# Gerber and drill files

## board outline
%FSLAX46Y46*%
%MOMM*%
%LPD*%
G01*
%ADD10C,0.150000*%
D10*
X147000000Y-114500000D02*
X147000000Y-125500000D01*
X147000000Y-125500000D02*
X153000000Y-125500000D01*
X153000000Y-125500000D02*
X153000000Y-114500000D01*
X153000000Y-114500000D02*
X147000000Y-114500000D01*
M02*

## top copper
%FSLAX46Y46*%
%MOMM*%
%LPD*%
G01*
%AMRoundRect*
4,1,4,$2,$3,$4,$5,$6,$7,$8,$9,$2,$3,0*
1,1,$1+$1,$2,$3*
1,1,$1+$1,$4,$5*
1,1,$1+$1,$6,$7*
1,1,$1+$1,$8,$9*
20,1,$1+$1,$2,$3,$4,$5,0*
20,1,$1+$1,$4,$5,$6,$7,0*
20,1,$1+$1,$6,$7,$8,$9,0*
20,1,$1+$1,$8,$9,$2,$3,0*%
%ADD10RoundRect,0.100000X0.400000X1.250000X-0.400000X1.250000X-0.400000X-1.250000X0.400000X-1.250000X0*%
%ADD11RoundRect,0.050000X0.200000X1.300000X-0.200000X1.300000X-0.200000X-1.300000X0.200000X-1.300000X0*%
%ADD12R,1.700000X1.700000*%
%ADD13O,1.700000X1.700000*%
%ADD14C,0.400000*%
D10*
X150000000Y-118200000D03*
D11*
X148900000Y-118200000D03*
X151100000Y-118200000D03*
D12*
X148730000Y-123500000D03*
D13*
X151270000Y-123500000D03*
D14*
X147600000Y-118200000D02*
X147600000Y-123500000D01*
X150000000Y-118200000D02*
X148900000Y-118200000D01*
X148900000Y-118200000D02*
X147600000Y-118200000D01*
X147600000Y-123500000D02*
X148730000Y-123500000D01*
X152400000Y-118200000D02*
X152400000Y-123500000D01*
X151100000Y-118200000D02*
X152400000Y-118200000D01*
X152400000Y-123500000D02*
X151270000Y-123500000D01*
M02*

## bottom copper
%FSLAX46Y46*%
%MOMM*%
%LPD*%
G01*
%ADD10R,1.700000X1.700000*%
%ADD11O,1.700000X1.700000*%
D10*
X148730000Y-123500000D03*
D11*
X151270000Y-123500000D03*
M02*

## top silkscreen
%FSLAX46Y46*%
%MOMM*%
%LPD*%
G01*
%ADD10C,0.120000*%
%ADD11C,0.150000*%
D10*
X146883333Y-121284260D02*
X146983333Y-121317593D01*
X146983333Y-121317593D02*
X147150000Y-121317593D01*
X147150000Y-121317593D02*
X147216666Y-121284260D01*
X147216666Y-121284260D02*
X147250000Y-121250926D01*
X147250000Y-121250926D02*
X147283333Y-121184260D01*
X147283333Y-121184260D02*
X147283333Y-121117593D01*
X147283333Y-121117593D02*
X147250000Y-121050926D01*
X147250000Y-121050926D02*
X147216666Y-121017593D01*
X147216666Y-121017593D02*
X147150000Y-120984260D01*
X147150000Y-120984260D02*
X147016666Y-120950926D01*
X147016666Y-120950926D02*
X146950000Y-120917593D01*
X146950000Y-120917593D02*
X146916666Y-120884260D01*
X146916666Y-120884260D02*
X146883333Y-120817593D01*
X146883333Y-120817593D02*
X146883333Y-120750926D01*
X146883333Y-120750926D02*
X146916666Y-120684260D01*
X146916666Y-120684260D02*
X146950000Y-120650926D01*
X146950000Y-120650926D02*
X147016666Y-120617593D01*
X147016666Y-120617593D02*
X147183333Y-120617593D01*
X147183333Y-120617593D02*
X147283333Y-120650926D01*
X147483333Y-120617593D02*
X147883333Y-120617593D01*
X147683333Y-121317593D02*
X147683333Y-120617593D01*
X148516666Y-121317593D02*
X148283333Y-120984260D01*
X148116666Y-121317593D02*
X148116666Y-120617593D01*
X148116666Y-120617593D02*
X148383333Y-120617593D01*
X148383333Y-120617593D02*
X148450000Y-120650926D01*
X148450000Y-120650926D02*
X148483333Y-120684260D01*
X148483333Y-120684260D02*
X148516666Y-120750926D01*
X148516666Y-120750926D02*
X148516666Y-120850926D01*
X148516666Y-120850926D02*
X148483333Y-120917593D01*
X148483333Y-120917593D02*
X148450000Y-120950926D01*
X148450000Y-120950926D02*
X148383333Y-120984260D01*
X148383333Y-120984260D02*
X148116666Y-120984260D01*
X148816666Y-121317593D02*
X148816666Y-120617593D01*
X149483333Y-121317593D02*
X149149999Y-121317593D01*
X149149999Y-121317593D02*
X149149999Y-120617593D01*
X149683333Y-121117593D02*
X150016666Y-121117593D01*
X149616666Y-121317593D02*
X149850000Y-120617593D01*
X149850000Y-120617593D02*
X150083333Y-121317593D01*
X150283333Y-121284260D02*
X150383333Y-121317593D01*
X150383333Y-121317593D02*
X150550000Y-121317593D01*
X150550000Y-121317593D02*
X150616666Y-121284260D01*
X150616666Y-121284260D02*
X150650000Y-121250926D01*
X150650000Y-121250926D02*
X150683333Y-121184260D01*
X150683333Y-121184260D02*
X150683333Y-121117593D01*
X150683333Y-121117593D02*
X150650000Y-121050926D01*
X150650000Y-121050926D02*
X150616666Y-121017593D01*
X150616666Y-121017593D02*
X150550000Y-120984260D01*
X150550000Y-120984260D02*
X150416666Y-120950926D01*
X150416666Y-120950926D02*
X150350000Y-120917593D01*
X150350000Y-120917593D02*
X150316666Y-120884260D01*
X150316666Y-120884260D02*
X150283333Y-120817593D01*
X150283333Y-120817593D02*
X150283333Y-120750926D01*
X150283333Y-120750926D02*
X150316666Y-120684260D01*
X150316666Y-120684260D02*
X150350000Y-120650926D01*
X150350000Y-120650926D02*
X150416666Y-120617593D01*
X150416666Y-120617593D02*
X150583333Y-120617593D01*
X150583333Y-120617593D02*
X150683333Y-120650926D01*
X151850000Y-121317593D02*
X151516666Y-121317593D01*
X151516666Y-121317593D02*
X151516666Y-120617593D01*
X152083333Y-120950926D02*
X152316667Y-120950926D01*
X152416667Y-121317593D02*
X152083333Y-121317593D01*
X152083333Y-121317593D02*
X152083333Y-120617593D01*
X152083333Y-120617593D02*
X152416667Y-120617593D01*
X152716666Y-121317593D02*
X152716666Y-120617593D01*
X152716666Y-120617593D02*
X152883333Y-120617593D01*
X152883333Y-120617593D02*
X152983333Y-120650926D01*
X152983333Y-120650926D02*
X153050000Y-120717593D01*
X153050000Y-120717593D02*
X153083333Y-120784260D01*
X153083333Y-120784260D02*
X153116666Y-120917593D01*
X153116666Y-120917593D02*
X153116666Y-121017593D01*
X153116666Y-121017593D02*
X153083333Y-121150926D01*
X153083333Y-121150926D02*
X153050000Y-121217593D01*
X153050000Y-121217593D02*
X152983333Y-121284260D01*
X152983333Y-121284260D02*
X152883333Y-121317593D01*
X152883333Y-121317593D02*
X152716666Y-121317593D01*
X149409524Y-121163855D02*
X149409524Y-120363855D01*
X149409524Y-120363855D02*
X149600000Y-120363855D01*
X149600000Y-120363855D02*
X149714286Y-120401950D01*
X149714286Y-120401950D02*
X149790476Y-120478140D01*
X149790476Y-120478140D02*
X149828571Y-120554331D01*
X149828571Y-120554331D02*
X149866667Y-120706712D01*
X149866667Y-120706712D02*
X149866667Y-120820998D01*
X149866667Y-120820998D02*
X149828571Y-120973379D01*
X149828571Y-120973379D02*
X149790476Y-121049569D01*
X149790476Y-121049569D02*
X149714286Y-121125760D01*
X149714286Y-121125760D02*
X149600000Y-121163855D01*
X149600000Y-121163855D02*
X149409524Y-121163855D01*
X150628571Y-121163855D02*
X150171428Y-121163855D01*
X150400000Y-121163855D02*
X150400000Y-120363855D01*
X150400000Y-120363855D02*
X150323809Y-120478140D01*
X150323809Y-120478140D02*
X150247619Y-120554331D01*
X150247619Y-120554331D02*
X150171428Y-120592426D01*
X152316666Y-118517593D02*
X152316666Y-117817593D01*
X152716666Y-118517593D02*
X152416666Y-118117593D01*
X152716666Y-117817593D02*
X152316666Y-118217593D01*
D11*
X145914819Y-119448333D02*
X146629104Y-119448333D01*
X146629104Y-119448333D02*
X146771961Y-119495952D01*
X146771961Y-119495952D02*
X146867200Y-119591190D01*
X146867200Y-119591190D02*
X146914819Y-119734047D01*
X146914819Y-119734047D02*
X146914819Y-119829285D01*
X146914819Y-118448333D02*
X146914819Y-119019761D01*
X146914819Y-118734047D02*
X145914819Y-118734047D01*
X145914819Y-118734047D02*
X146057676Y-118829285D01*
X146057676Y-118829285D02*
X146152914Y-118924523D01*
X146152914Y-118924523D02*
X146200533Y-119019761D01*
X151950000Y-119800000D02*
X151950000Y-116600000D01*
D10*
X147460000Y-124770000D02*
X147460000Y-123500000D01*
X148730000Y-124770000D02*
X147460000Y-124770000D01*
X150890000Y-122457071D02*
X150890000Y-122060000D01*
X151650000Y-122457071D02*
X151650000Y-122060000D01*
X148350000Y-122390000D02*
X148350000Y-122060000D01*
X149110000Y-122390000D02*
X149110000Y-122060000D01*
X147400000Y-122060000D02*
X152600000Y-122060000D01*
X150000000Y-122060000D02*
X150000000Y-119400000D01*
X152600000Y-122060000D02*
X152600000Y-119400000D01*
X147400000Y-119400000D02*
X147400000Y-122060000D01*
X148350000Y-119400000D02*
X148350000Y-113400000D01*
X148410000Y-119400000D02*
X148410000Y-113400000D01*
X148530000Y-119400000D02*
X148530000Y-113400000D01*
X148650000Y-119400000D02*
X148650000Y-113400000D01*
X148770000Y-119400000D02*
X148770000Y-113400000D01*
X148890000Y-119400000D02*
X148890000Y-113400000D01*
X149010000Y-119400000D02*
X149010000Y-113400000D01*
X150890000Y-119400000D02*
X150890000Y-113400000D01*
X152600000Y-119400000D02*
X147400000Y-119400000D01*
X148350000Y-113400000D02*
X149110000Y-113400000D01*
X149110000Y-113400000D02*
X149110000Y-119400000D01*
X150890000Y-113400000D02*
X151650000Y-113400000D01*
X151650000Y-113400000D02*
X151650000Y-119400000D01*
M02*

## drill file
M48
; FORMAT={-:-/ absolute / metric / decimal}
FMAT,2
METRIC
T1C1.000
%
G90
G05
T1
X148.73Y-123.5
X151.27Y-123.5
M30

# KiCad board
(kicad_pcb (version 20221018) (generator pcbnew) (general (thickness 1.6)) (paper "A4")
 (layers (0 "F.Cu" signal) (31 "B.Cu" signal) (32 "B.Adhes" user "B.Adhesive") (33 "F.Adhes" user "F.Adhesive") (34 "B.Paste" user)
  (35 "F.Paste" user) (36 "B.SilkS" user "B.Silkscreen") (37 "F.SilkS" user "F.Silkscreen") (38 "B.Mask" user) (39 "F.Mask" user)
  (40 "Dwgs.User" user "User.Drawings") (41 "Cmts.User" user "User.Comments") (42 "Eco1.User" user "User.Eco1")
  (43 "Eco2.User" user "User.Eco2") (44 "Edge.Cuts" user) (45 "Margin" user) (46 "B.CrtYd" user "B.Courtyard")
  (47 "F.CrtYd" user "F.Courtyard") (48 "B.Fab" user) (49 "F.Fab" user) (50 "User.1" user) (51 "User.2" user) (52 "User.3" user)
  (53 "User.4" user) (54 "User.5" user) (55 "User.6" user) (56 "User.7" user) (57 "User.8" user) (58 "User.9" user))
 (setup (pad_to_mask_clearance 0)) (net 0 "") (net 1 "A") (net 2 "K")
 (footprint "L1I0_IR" (layer "F.Cu") (at 150 118.2 180)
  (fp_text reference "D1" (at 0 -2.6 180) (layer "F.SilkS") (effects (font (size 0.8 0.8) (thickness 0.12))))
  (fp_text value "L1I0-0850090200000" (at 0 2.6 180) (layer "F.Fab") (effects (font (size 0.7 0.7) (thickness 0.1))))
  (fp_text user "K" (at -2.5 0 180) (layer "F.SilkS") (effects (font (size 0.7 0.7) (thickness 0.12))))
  (fp_line (start -1.95 -1.6) (end -1.95 1.6) (stroke (width 0.15) (type solid)) (layer "F.SilkS"))
  (pad "1" smd roundrect (at 0 0 180) (size 1 2.7) (layers "F.Cu" "F.Paste" "F.Mask") (roundrect_rratio 0.1) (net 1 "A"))
  (pad "1" smd roundrect (at 1.1 0 180) (size 0.5 2.7) (layers "F.Cu" "F.Paste" "F.Mask") (roundrect_rratio 0.1) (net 1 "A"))
  (pad "2" smd roundrect (at -1.1 0 180) (size 0.5 2.7) (layers "F.Cu" "F.Paste" "F.Mask") (roundrect_rratio 0.1) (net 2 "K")))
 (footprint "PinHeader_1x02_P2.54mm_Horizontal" (layer "F.Cu") (at 148.73 123.5 90)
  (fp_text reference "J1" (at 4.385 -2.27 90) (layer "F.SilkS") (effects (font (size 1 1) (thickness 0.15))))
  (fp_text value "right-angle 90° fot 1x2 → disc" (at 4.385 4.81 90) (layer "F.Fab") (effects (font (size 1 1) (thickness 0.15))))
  (fp_line (start -1.27 -1.27) (end 0 -1.27) (stroke (width 0.12) (type solid)) (layer "F.SilkS"))
  (fp_line (start -1.27 0) (end -1.27 -1.27) (stroke (width 0.12) (type solid)) (layer "F.SilkS"))
  (fp_line (start 1.042929 2.16) (end 1.44 2.16) (stroke (width 0.12) (type solid)) (layer "F.SilkS"))
  (fp_line (start 1.042929 2.92) (end 1.44 2.92) (stroke (width 0.12) (type solid)) (layer "F.SilkS"))
  (fp_line (start 1.11 -0.38) (end 1.44 -0.38) (stroke (width 0.12) (type solid)) (layer "F.SilkS"))
  (fp_line (start 1.11 0.38) (end 1.44 0.38) (stroke (width 0.12) (type solid)) (layer "F.SilkS"))
  (fp_line (start 1.44 -1.33) (end 1.44 3.87) (stroke (width 0.12) (type solid)) (layer "F.SilkS"))
  (fp_line (start 1.44 1.27) (end 4.1 1.27) (stroke (width 0.12) (type solid)) (layer "F.SilkS"))
  (fp_line (start 1.44 3.87) (end 4.1 3.87) (stroke (width 0.12) (type solid)) (layer "F.SilkS"))
  (fp_line (start 4.1 -1.33) (end 1.44 -1.33) (stroke (width 0.12) (type solid)) (layer "F.SilkS"))
  (fp_line (start 4.1 -0.38) (end 10.1 -0.38) (stroke (width 0.12) (type solid)) (layer "F.SilkS"))
  (fp_line (start 4.1 -0.32) (end 10.1 -0.32) (stroke (width 0.12) (type solid)) (layer "F.SilkS"))
  (fp_line (start 4.1 -0.2) (end 10.1 -0.2) (stroke (width 0.12) (type solid)) (layer "F.SilkS"))
  (fp_line (start 4.1 -0.08) (end 10.1 -0.08) (stroke (width 0.12) (type solid)) (layer "F.SilkS"))
  (fp_line (start 4.1 0.04) (end 10.1 0.04) (stroke (width 0.12) (type solid)) (layer "F.SilkS"))
  (fp_line (start 4.1 0.16) (end 10.1 0.16) (stroke (width 0.12) (type solid)) (layer "F.SilkS"))
  (fp_line (start 4.1 0.28) (end 10.1 0.28) (stroke (width 0.12) (type solid)) (layer "F.SilkS"))
  (fp_line (start 4.1 2.16) (end 10.1 2.16) (stroke (width 0.12) (type solid)) (layer "F.SilkS"))
  (fp_line (start 4.1 3.87) (end 4.1 -1.33) (stroke (width 0.12) (type solid)) (layer "F.SilkS"))
  (fp_line (start 10.1 -0.38) (end 10.1 0.38) (stroke (width 0.12) (type solid)) (layer "F.SilkS"))
  (fp_line (start 10.1 0.38) (end 4.1 0.38) (stroke (width 0.12) (type solid)) (layer "F.SilkS"))
  (fp_line (start 10.1 2.16) (end 10.1 2.92) (stroke (width 0.12) (type solid)) (layer "F.SilkS"))
  (fp_line (start 10.1 2.92) (end 4.1 2.92) (stroke (width 0.12) (type solid)) (layer "F.SilkS"))
  (pad "1" thru_hole rect (at 0 0 90) (size 1.7 1.7) (drill 1) (layers "*.Cu" "*.Mask") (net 1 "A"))
  (pad "2" thru_hole oval (at 0 2.54 90) (size 1.7 1.7) (drill 1) (layers "*.Cu" "*.Mask") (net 2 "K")))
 (gr_line (start 147 114.5) (end 147 125.5) (stroke (width 0.15) (type default)) (layer "Edge.Cuts"))
 (gr_line (start 147 125.5) (end 153 125.5) (stroke (width 0.15) (type default)) (layer "Edge.Cuts"))
 (gr_line (start 153 125.5) (end 153 114.5) (stroke (width 0.15) (type default)) (layer "Edge.Cuts"))
 (gr_line (start 153 114.5) (end 147 114.5) (stroke (width 0.15) (type default)) (layer "Edge.Cuts"))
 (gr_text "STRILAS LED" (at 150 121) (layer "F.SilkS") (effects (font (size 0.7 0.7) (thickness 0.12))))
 (segment (start 147.6 118.2) (end 147.6 123.5) (width 0.4) (layer "F.Cu") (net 1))
 (segment (start 150 118.2) (end 148.9 118.2) (width 0.4) (layer "F.Cu") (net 1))
 (segment (start 148.9 118.2) (end 147.6 118.2) (width 0.4) (layer "F.Cu") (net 1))
 (segment (start 147.6 123.5) (end 148.73 123.5) (width 0.4) (layer "F.Cu") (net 1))
 (segment (start 152.4 118.2) (end 152.4 123.5) (width 0.4) (layer "F.Cu") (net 2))
 (segment (start 151.1 118.2) (end 152.4 118.2) (width 0.4) (layer "F.Cu") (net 2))
 (segment (start 152.4 123.5) (end 151.27 123.5) (width 0.4) (layer "F.Cu") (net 2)))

